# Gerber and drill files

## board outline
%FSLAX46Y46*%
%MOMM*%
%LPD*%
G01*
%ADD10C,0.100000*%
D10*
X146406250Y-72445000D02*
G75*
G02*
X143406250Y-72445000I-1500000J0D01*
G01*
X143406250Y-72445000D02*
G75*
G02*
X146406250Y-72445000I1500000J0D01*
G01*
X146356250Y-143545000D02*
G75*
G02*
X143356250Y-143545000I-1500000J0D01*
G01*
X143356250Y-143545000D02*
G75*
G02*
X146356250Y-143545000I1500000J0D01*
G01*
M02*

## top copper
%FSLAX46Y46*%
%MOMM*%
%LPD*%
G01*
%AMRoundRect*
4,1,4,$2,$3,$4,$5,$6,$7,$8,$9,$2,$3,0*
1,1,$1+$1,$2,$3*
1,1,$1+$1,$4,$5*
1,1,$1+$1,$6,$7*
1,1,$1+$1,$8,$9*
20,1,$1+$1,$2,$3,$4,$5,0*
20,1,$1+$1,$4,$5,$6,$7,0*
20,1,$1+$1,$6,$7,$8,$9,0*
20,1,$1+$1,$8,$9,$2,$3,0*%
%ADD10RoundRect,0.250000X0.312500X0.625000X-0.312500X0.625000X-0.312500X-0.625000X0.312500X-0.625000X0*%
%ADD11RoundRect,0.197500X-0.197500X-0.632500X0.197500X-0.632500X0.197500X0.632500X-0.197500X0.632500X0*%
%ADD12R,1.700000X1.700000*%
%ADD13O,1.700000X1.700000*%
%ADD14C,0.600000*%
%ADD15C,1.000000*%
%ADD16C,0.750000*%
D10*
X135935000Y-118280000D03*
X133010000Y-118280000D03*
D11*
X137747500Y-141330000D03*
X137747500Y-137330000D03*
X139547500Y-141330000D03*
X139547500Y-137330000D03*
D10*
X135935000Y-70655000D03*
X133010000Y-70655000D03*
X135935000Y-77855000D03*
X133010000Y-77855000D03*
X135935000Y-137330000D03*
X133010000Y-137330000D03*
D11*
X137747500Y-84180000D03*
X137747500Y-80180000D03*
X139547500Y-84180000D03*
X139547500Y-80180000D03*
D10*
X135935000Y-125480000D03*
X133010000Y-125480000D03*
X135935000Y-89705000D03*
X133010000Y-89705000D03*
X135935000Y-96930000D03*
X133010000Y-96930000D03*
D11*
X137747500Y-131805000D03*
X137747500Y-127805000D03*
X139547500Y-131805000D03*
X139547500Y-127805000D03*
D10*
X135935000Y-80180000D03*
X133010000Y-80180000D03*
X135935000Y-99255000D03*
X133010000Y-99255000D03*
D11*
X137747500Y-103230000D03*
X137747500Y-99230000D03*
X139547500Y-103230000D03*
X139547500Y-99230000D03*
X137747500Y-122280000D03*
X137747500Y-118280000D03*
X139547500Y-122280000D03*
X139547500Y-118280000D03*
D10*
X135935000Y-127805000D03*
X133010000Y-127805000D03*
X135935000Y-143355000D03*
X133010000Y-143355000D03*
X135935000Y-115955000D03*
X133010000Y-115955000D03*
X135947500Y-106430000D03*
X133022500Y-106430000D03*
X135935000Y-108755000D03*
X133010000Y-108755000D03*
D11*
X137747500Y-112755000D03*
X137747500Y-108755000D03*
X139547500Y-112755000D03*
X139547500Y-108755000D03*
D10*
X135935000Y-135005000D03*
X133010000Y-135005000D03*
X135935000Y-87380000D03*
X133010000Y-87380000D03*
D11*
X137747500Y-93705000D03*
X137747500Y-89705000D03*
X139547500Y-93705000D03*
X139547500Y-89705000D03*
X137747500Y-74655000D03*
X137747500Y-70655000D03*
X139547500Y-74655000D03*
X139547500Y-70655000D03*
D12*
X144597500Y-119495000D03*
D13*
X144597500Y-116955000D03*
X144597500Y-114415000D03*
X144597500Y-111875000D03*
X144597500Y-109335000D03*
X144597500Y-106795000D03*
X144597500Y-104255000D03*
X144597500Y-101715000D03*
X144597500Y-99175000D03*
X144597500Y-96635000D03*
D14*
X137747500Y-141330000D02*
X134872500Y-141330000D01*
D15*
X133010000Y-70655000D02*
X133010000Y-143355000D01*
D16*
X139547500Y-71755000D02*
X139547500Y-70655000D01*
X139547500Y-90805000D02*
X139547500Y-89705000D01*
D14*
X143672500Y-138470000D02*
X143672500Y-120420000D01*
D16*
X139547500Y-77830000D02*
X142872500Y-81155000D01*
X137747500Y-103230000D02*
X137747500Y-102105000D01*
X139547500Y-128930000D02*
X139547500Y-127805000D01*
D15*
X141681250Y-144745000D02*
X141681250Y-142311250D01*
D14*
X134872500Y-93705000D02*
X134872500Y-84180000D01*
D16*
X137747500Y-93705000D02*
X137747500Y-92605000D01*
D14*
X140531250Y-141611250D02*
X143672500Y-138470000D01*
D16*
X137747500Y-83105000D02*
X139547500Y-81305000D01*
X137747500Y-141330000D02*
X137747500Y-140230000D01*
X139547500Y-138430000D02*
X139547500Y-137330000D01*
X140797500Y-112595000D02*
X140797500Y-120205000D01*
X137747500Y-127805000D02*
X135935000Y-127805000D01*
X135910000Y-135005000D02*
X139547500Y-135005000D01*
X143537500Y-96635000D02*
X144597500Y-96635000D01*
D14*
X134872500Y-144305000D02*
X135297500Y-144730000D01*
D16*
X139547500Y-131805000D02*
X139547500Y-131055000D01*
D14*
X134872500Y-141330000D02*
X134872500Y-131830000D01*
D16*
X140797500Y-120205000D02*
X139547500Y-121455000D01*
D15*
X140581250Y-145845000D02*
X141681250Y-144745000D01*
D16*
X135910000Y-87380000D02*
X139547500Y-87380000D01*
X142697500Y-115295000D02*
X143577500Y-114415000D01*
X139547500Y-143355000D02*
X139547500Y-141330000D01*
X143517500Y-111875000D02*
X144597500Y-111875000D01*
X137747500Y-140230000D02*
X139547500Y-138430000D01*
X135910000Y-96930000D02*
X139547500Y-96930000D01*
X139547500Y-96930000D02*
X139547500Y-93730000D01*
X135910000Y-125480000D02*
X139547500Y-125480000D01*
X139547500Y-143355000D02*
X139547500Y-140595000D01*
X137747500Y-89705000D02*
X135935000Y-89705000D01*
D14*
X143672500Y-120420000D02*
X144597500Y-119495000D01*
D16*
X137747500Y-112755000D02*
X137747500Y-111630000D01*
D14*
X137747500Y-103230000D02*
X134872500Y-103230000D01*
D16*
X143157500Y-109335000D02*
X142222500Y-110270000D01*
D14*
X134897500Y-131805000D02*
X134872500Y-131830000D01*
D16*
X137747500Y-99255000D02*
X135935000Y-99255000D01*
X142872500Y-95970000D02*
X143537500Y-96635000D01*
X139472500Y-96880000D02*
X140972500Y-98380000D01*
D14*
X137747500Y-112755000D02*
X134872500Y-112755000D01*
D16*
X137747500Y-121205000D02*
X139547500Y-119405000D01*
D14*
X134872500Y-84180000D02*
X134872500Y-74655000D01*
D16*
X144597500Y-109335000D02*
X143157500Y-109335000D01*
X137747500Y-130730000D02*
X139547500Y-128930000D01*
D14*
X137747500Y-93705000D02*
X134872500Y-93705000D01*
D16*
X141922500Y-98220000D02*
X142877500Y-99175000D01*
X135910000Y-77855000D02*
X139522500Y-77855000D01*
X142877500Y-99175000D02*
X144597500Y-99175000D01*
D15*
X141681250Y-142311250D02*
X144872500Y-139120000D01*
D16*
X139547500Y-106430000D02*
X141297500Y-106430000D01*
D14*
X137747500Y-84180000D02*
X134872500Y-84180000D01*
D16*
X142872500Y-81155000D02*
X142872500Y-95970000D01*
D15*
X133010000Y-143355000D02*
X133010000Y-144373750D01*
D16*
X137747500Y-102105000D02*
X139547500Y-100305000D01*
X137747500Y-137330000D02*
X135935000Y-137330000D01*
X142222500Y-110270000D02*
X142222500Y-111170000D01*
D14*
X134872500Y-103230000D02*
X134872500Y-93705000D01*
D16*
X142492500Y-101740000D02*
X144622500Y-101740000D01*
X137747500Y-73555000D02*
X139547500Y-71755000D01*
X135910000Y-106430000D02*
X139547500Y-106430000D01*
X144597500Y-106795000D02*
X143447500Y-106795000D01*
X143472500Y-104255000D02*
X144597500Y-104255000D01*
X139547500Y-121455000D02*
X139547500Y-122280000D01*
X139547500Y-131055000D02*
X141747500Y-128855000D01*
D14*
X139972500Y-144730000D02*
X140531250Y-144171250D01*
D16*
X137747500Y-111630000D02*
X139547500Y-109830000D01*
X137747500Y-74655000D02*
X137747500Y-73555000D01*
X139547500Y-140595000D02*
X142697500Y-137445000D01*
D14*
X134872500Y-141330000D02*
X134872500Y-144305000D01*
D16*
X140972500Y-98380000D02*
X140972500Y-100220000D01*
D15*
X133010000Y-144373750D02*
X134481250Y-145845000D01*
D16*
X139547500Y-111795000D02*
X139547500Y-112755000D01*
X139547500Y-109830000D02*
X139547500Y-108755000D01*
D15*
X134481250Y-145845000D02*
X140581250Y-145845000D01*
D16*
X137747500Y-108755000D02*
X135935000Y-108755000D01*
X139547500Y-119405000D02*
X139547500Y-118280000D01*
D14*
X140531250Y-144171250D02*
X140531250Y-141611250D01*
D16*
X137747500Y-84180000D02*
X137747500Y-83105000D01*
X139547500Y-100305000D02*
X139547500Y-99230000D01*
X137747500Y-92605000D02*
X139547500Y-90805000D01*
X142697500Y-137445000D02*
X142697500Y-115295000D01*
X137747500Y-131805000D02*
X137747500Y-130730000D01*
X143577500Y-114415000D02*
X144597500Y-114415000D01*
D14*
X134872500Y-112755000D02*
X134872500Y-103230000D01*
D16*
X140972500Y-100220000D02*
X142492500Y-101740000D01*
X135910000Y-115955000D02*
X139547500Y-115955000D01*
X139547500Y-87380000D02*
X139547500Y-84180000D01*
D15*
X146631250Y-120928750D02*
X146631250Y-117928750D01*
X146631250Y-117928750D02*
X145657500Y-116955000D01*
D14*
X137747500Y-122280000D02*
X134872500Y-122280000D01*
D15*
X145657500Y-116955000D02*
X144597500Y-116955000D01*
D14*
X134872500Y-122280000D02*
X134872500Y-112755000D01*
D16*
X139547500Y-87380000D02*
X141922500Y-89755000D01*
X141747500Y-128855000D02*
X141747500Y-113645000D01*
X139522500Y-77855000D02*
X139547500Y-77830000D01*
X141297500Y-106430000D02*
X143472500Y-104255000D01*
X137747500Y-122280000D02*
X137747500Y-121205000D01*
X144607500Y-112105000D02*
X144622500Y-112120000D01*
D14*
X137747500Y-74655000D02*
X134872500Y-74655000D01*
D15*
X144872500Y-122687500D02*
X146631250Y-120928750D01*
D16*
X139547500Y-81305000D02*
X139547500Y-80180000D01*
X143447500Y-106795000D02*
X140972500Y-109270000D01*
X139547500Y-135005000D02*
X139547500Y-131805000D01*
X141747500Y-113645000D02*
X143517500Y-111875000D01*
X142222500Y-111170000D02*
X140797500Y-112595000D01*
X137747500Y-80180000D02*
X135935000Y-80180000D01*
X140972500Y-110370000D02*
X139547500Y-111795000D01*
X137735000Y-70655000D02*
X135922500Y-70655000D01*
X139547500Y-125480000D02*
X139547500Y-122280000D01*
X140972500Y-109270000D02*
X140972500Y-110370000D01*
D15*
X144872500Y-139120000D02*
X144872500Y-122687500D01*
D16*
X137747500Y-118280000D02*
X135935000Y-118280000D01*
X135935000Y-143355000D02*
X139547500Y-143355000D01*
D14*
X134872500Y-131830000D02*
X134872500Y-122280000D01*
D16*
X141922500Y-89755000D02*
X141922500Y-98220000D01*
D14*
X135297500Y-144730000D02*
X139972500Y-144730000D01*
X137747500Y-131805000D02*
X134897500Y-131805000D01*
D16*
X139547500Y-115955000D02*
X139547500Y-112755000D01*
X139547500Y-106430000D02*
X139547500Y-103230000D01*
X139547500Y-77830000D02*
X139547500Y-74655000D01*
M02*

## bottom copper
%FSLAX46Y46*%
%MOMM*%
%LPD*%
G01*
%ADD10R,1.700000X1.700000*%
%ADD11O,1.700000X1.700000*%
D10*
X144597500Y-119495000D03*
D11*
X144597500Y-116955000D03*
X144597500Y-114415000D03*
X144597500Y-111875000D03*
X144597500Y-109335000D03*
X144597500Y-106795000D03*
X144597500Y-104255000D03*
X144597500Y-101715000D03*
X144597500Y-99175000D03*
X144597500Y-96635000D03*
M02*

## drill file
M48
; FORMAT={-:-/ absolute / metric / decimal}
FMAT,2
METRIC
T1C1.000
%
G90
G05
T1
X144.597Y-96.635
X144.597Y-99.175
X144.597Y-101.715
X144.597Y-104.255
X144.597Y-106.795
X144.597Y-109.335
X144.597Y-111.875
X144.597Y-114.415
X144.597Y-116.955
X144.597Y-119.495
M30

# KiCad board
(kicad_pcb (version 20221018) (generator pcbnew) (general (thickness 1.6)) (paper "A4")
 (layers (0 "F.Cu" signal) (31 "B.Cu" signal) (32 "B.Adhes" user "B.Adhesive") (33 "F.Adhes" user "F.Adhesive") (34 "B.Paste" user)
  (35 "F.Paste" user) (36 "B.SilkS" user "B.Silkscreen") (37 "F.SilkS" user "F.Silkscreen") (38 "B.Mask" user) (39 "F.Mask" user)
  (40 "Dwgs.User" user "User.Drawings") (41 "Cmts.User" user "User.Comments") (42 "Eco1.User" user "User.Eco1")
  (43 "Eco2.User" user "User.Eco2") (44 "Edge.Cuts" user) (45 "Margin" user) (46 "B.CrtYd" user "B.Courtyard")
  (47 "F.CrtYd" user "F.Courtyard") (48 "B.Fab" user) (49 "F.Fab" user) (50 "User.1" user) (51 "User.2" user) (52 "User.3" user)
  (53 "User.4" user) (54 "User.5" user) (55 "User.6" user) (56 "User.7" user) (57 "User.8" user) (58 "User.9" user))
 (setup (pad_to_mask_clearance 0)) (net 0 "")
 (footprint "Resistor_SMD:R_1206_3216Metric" (layer "F.Cu") (at 134.4725 118.28 180)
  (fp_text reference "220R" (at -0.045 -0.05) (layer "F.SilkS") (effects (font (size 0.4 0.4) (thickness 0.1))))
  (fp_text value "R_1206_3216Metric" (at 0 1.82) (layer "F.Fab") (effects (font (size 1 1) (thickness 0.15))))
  (pad "1" smd roundrect (at -1.4625 0 180) (size 1.125 1.75) (layers "F.Cu" "F.Paste" "F.Mask") (roundrect_rratio 0.2222222222))
  (pad "2" smd roundrect (at 1.4625 0 180) (size 1.125 1.75) (layers "F.Cu" "F.Paste" "F.Mask") (roundrect_rratio 0.2222222222)))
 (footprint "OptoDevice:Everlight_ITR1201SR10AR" (layer "F.Cu") (at 138.6475 139.33)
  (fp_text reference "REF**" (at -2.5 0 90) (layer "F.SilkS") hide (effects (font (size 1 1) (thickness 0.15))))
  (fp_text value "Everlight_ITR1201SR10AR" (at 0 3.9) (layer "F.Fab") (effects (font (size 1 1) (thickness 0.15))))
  (pad "1" smd roundrect (at -0.9 2) (size 0.79 1.66) (layers "F.Cu" "F.Paste" "F.Mask") (roundrect_rratio 0.25))
  (pad "2" smd roundrect (at -0.9 -2) (size 0.79 1.66) (layers "F.Cu" "F.Paste" "F.Mask") (roundrect_rratio 0.25))
  (pad "3" smd roundrect (at 0.9 2) (size 0.79 1.66) (layers "F.Cu" "F.Paste" "F.Mask") (roundrect_rratio 0.25))
  (pad "4" smd roundrect (at 0.9 -2) (size 0.79 1.66) (layers "F.Cu" "F.Paste" "F.Mask") (roundrect_rratio 0.25)))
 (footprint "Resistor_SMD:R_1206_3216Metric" (layer "F.Cu") (at 134.4725 70.655 180)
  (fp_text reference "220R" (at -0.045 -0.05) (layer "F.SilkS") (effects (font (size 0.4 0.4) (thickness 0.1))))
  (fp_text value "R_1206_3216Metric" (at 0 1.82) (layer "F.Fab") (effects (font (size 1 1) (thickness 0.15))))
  (pad "1" smd roundrect (at -1.4625 0 180) (size 1.125 1.75) (layers "F.Cu" "F.Paste" "F.Mask") (roundrect_rratio 0.2222222222))
  (pad "2" smd roundrect (at 1.4625 0 180) (size 1.125 1.75) (layers "F.Cu" "F.Paste" "F.Mask") (roundrect_rratio 0.2222222222)))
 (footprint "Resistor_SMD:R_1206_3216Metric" (layer "F.Cu") (at 134.4725 77.855 180)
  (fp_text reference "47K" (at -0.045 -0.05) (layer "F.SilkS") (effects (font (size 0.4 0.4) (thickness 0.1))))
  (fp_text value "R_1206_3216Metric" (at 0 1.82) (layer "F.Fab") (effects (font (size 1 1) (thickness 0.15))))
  (pad "1" smd roundrect (at -1.4625 0 180) (size 1.125 1.75) (layers "F.Cu" "F.Paste" "F.Mask") (roundrect_rratio 0.2222222222))
  (pad "2" smd roundrect (at 1.4625 0 180) (size 1.125 1.75) (layers "F.Cu" "F.Paste" "F.Mask") (roundrect_rratio 0.2222222222)))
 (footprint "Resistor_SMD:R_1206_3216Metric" (layer "F.Cu") (at 134.4725 137.33 180)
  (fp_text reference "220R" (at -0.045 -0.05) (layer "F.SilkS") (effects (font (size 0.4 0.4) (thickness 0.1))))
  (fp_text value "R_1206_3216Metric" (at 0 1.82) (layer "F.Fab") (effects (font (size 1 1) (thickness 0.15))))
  (pad "1" smd roundrect (at -1.4625 0 180) (size 1.125 1.75) (layers "F.Cu" "F.Paste" "F.Mask") (roundrect_rratio 0.2222222222))
  (pad "2" smd roundrect (at 1.4625 0 180) (size 1.125 1.75) (layers "F.Cu" "F.Paste" "F.Mask") (roundrect_rratio 0.2222222222)))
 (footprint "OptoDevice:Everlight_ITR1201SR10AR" (layer "F.Cu") (at 138.6475 82.18)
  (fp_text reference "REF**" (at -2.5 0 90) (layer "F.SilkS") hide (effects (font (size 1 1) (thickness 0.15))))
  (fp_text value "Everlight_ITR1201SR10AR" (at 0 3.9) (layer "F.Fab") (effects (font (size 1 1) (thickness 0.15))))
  (pad "1" smd roundrect (at -0.9 2) (size 0.79 1.66) (layers "F.Cu" "F.Paste" "F.Mask") (roundrect_rratio 0.25))
  (pad "2" smd roundrect (at -0.9 -2) (size 0.79 1.66) (layers "F.Cu" "F.Paste" "F.Mask") (roundrect_rratio 0.25))
  (pad "3" smd roundrect (at 0.9 2) (size 0.79 1.66) (layers "F.Cu" "F.Paste" "F.Mask") (roundrect_rratio 0.25))
  (pad "4" smd roundrect (at 0.9 -2) (size 0.79 1.66) (layers "F.Cu" "F.Paste" "F.Mask") (roundrect_rratio 0.25)))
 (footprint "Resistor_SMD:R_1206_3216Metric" (layer "F.Cu") (at 134.4725 125.48 180)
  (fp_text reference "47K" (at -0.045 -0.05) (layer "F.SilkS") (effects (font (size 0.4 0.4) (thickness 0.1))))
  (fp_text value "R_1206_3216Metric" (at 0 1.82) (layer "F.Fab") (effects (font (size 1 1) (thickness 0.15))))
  (pad "1" smd roundrect (at -1.4625 0 180) (size 1.125 1.75) (layers "F.Cu" "F.Paste" "F.Mask") (roundrect_rratio 0.2222222222))
  (pad "2" smd roundrect (at 1.4625 0 180) (size 1.125 1.75) (layers "F.Cu" "F.Paste" "F.Mask") (roundrect_rratio 0.2222222222)))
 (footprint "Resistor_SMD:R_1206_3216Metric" (layer "F.Cu") (at 134.4725 89.705 180)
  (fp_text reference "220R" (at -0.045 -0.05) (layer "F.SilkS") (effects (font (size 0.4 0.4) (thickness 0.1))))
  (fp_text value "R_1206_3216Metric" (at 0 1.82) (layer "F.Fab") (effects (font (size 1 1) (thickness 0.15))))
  (pad "1" smd roundrect (at -1.4625 0 180) (size 1.125 1.75) (layers "F.Cu" "F.Paste" "F.Mask") (roundrect_rratio 0.2222222222))
  (pad "2" smd roundrect (at 1.4625 0 180) (size 1.125 1.75) (layers "F.Cu" "F.Paste" "F.Mask") (roundrect_rratio 0.2222222222)))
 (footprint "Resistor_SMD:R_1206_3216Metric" (layer "F.Cu") (at 134.4725 96.93 180)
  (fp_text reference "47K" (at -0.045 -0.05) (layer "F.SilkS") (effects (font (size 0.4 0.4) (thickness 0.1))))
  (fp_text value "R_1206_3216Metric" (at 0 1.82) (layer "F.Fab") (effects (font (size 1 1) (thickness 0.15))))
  (pad "1" smd roundrect (at -1.4625 0 180) (size 1.125 1.75) (layers "F.Cu" "F.Paste" "F.Mask") (roundrect_rratio 0.2222222222))
  (pad "2" smd roundrect (at 1.4625 0 180) (size 1.125 1.75) (layers "F.Cu" "F.Paste" "F.Mask") (roundrect_rratio 0.2222222222)))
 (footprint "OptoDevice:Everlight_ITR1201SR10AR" (layer "F.Cu") (at 138.6475 129.805)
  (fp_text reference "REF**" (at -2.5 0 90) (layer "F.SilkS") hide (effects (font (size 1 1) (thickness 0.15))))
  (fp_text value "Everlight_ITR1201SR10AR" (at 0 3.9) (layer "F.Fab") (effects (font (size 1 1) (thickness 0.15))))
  (pad "1" smd roundrect (at -0.9 2) (size 0.79 1.66) (layers "F.Cu" "F.Paste" "F.Mask") (roundrect_rratio 0.25))
  (pad "2" smd roundrect (at -0.9 -2) (size 0.79 1.66) (layers "F.Cu" "F.Paste" "F.Mask") (roundrect_rratio 0.25))
  (pad "3" smd roundrect (at 0.9 2) (size 0.79 1.66) (layers "F.Cu" "F.Paste" "F.Mask") (roundrect_rratio 0.25))
  (pad "4" smd roundrect (at 0.9 -2) (size 0.79 1.66) (layers "F.Cu" "F.Paste" "F.Mask") (roundrect_rratio 0.25)))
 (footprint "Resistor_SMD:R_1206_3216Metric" (layer "F.Cu") (at 134.4725 80.18 180)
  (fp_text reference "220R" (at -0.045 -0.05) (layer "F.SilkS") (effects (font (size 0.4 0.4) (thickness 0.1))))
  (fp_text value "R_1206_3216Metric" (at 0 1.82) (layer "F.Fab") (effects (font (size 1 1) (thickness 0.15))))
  (pad "1" smd roundrect (at -1.4625 0 180) (size 1.125 1.75) (layers "F.Cu" "F.Paste" "F.Mask") (roundrect_rratio 0.2222222222))
  (pad "2" smd roundrect (at 1.4625 0 180) (size 1.125 1.75) (layers "F.Cu" "F.Paste" "F.Mask") (roundrect_rratio 0.2222222222)))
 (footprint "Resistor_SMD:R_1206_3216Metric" (layer "F.Cu") (at 134.4725 99.255 180)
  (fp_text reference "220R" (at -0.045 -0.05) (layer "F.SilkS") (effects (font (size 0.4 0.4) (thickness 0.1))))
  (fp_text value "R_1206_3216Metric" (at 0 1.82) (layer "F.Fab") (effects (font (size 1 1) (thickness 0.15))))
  (pad "1" smd roundrect (at -1.4625 0 180) (size 1.125 1.75) (layers "F.Cu" "F.Paste" "F.Mask") (roundrect_rratio 0.2222222222))
  (pad "2" smd roundrect (at 1.4625 0 180) (size 1.125 1.75) (layers "F.Cu" "F.Paste" "F.Mask") (roundrect_rratio 0.2222222222)))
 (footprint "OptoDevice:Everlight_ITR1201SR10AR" (layer "F.Cu") (at 138.6475 101.23)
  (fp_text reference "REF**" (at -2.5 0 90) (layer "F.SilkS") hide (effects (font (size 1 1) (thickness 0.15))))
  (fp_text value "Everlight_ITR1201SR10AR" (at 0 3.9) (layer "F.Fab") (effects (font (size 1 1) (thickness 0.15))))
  (pad "1" smd roundrect (at -0.9 2) (size 0.79 1.66) (layers "F.Cu" "F.Paste" "F.Mask") (roundrect_rratio 0.25))
  (pad "2" smd roundrect (at -0.9 -2) (size 0.79 1.66) (layers "F.Cu" "F.Paste" "F.Mask") (roundrect_rratio 0.25))
  (pad "3" smd roundrect (at 0.9 2) (size 0.79 1.66) (layers "F.Cu" "F.Paste" "F.Mask") (roundrect_rratio 0.25))
  (pad "4" smd roundrect (at 0.9 -2) (size 0.79 1.66) (layers "F.Cu" "F.Paste" "F.Mask") (roundrect_rratio 0.25)))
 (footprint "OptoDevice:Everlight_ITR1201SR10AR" (layer "F.Cu") (at 138.6475 120.28)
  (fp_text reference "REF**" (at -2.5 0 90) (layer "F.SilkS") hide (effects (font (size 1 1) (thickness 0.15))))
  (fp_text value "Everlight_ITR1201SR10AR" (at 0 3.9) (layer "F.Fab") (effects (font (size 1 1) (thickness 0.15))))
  (pad "1" smd roundrect (at -0.9 2) (size 0.79 1.66) (layers "F.Cu" "F.Paste" "F.Mask") (roundrect_rratio 0.25))
  (pad "2" smd roundrect (at -0.9 -2) (size 0.79 1.66) (layers "F.Cu" "F.Paste" "F.Mask") (roundrect_rratio 0.25))
  (pad "3" smd roundrect (at 0.9 2) (size 0.79 1.66) (layers "F.Cu" "F.Paste" "F.Mask") (roundrect_rratio 0.25))
  (pad "4" smd roundrect (at 0.9 -2) (size 0.79 1.66) (layers "F.Cu" "F.Paste" "F.Mask") (roundrect_rratio 0.25)))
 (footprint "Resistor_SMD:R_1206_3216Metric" (layer "F.Cu") (at 134.4725 127.805 180)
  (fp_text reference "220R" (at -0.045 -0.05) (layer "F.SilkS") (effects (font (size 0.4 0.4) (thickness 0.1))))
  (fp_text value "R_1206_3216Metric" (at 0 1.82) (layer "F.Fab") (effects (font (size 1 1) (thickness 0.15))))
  (pad "1" smd roundrect (at -1.4625 0 180) (size 1.125 1.75) (layers "F.Cu" "F.Paste" "F.Mask") (roundrect_rratio 0.2222222222))
  (pad "2" smd roundrect (at 1.4625 0 180) (size 1.125 1.75) (layers "F.Cu" "F.Paste" "F.Mask") (roundrect_rratio 0.2222222222)))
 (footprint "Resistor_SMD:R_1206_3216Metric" (layer "F.Cu") (at 134.4725 143.355 180)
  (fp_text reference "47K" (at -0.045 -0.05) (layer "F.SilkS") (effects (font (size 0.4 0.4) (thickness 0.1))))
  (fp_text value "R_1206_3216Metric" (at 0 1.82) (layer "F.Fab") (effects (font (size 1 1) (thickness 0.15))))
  (pad "1" smd roundrect (at -1.4625 0 180) (size 1.125 1.75) (layers "F.Cu" "F.Paste" "F.Mask") (roundrect_rratio 0.2222222222))
  (pad "2" smd roundrect (at 1.4625 0 180) (size 1.125 1.75) (layers "F.Cu" "F.Paste" "F.Mask") (roundrect_rratio 0.2222222222)))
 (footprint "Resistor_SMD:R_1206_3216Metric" (layer "F.Cu") (at 134.4725 115.955 180)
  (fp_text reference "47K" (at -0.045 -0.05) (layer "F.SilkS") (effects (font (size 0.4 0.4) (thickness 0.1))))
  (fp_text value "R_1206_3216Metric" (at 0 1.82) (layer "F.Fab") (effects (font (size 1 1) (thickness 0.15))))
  (pad "1" smd roundrect (at -1.4625 0 180) (size 1.125 1.75) (layers "F.Cu" "F.Paste" "F.Mask") (roundrect_rratio 0.2222222222))
  (pad "2" smd roundrect (at 1.4625 0 180) (size 1.125 1.75) (layers "F.Cu" "F.Paste" "F.Mask") (roundrect_rratio 0.2222222222)))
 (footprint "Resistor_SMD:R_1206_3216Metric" (layer "F.Cu") (at 134.485 106.43 180)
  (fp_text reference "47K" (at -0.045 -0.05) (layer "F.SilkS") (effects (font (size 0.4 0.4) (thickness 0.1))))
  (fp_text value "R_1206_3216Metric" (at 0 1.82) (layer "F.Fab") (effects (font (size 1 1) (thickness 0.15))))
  (pad "1" smd roundrect (at -1.4625 0 180) (size 1.125 1.75) (layers "F.Cu" "F.Paste" "F.Mask") (roundrect_rratio 0.2222222222))
  (pad "2" smd roundrect (at 1.4625 0 180) (size 1.125 1.75) (layers "F.Cu" "F.Paste" "F.Mask") (roundrect_rratio 0.2222222222)))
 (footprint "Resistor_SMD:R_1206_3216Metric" (layer "F.Cu") (at 134.4725 108.755 180)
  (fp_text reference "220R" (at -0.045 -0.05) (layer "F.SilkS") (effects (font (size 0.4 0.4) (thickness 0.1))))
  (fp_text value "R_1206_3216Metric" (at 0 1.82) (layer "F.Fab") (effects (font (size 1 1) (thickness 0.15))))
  (pad "1" smd roundrect (at -1.4625 0 180) (size 1.125 1.75) (layers "F.Cu" "F.Paste" "F.Mask") (roundrect_rratio 0.2222222222))
  (pad "2" smd roundrect (at 1.4625 0 180) (size 1.125 1.75) (layers "F.Cu" "F.Paste" "F.Mask") (roundrect_rratio 0.2222222222)))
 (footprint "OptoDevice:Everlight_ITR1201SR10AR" (layer "F.Cu") (at 138.6475 110.755)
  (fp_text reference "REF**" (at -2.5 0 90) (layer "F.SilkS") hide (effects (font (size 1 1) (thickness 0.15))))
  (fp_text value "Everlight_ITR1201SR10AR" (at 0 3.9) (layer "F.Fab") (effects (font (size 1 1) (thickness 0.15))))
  (pad "1" smd roundrect (at -0.9 2) (size 0.79 1.66) (layers "F.Cu" "F.Paste" "F.Mask") (roundrect_rratio 0.25))
  (pad "2" smd roundrect (at -0.9 -2) (size 0.79 1.66) (layers "F.Cu" "F.Paste" "F.Mask") (roundrect_rratio 0.25))
  (pad "3" smd roundrect (at 0.9 2) (size 0.79 1.66) (layers "F.Cu" "F.Paste" "F.Mask") (roundrect_rratio 0.25))
  (pad "4" smd roundrect (at 0.9 -2) (size 0.79 1.66) (layers "F.Cu" "F.Paste" "F.Mask") (roundrect_rratio 0.25)))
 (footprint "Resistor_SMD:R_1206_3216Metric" (layer "F.Cu") (at 134.4725 135.005 180)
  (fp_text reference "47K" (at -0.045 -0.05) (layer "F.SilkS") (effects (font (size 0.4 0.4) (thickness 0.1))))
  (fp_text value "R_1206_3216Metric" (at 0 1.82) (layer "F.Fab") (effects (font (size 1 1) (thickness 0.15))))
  (pad "1" smd roundrect (at -1.4625 0 180) (size 1.125 1.75) (layers "F.Cu" "F.Paste" "F.Mask") (roundrect_rratio 0.2222222222))
  (pad "2" smd roundrect (at 1.4625 0 180) (size 1.125 1.75) (layers "F.Cu" "F.Paste" "F.Mask") (roundrect_rratio 0.2222222222)))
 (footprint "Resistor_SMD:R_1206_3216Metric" (layer "F.Cu") (at 134.4725 87.38 180)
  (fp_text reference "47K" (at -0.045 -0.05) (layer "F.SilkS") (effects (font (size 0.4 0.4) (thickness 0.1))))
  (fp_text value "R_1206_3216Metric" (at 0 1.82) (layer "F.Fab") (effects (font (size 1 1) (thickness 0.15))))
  (pad "1" smd roundrect (at -1.4625 0 180) (size 1.125 1.75) (layers "F.Cu" "F.Paste" "F.Mask") (roundrect_rratio 0.2222222222))
  (pad "2" smd roundrect (at 1.4625 0 180) (size 1.125 1.75) (layers "F.Cu" "F.Paste" "F.Mask") (roundrect_rratio 0.2222222222)))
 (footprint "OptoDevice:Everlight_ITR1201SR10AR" (layer "F.Cu") (at 138.6475 91.705)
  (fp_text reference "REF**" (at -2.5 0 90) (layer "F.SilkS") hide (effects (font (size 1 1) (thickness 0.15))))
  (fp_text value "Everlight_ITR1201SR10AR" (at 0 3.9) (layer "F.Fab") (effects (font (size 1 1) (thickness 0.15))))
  (pad "1" smd roundrect (at -0.9 2) (size 0.79 1.66) (layers "F.Cu" "F.Paste" "F.Mask") (roundrect_rratio 0.25))
  (pad "2" smd roundrect (at -0.9 -2) (size 0.79 1.66) (layers "F.Cu" "F.Paste" "F.Mask") (roundrect_rratio 0.25))
  (pad "3" smd roundrect (at 0.9 2) (size 0.79 1.66) (layers "F.Cu" "F.Paste" "F.Mask") (roundrect_rratio 0.25))
  (pad "4" smd roundrect (at 0.9 -2) (size 0.79 1.66) (layers "F.Cu" "F.Paste" "F.Mask") (roundrect_rratio 0.25)))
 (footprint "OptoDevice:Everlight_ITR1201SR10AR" (layer "F.Cu") (at 138.6475 72.655)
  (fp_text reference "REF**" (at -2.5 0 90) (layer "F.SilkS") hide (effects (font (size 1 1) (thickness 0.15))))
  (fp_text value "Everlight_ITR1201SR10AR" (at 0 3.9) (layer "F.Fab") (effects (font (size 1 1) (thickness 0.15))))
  (pad "1" smd roundrect (at -0.9 2) (size 0.79 1.66) (layers "F.Cu" "F.Paste" "F.Mask") (roundrect_rratio 0.25))
  (pad "2" smd roundrect (at -0.9 -2) (size 0.79 1.66) (layers "F.Cu" "F.Paste" "F.Mask") (roundrect_rratio 0.25))
  (pad "3" smd roundrect (at 0.9 2) (size 0.79 1.66) (layers "F.Cu" "F.Paste" "F.Mask") (roundrect_rratio 0.25))
  (pad "4" smd roundrect (at 0.9 -2) (size 0.79 1.66) (layers "F.Cu" "F.Paste" "F.Mask") (roundrect_rratio 0.25)))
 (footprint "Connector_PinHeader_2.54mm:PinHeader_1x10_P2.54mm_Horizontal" (layer "B.Cu") (at 144.5975 119.495)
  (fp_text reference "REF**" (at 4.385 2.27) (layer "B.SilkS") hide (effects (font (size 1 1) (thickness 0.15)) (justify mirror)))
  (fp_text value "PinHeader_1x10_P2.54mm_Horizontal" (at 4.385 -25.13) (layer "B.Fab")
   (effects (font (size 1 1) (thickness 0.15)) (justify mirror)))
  (pad "1" thru_hole rect (at 0 0) (size 1.7 1.7) (drill 1) (layers "*.Cu" "*.Mask"))
  (pad "2" thru_hole oval (at 0 -2.54) (size 1.7 1.7) (drill 1) (layers "*.Cu" "*.Mask"))
  (pad "3" thru_hole oval (at 0 -5.08) (size 1.7 1.7) (drill 1) (layers "*.Cu" "*.Mask"))
  (pad "4" thru_hole oval (at 0 -7.62) (size 1.7 1.7) (drill 1) (layers "*.Cu" "*.Mask"))
  (pad "5" thru_hole oval (at 0 -10.16) (size 1.7 1.7) (drill 1) (layers "*.Cu" "*.Mask"))
  (pad "6" thru_hole oval (at 0 -12.7) (size 1.7 1.7) (drill 1) (layers "*.Cu" "*.Mask"))
  (pad "7" thru_hole oval (at 0 -15.24) (size 1.7 1.7) (drill 1) (layers "*.Cu" "*.Mask"))
  (pad "8" thru_hole oval (at 0 -17.78) (size 1.7 1.7) (drill 1) (layers "*.Cu" "*.Mask"))
  (pad "9" thru_hole oval (at 0 -20.32) (size 1.7 1.7) (drill 1) (layers "*.Cu" "*.Mask"))
  (pad "10" thru_hole oval (at 0 -22.86) (size 1.7 1.7) (drill 1) (layers "*.Cu" "*.Mask")))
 (gr_circle (center 144.90625 72.445) (end 143.40625 72.445) (stroke (width 0.1) (type solid)) (fill none) (layer "Edge.Cuts"))
 (gr_circle (center 144.85625 143.545) (end 146.35625 143.545) (stroke (width 0.1) (type solid)) (fill none) (layer "Edge.Cuts"))
 (segment (start 137.7475 141.33) (end 134.8725 141.33) (width 0.6) (layer "F.Cu") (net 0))
 (segment (start 133.01 70.655) (end 133.01 143.355) (width 1) (layer "F.Cu") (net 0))
 (segment (start 139.5475 71.755) (end 139.5475 70.655) (width 0.75) (layer "F.Cu") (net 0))
 (segment (start 139.5475 90.805) (end 139.5475 89.705) (width 0.75) (layer "F.Cu") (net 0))
 (segment (start 143.6725 138.47) (end 143.6725 120.42) (width 0.6) (layer "F.Cu") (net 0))
 (segment (start 139.5475 77.83) (end 142.8725 81.155) (width 0.75) (layer "F.Cu") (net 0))
 (segment (start 137.7475 103.23) (end 137.7475 102.105) (width 0.75) (layer "F.Cu") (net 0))
 (segment (start 139.5475 128.93) (end 139.5475 127.805) (width 0.75) (layer "F.Cu") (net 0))
 (segment (start 141.68125 144.745) (end 141.68125 142.31125) (width 1) (layer "F.Cu") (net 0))
 (segment (start 134.8725 93.705) (end 134.8725 84.18) (width 0.6) (layer "F.Cu") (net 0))
 (segment (start 137.7475 93.705) (end 137.7475 92.605) (width 0.75) (layer "F.Cu") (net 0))
 (segment (start 140.53125 141.61125) (end 143.6725 138.47) (width 0.6) (layer "F.Cu") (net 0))
 (segment (start 137.7475 83.105) (end 139.5475 81.305) (width 0.75) (layer "F.Cu") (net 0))
 (segment (start 137.7475 141.33) (end 137.7475 140.23) (width 0.75) (layer "F.Cu") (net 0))
 (segment (start 139.5475 138.43) (end 139.5475 137.33) (width 0.75) (layer "F.Cu") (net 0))
 (segment (start 140.7975 112.595) (end 140.7975 120.205) (width 0.75) (layer "F.Cu") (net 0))
 (segment (start 137.7475 127.805) (end 135.935 127.805) (width 0.75) (layer "F.Cu") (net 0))
 (segment (start 135.91 135.005) (end 139.5475 135.005) (width 0.75) (layer "F.Cu") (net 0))
 (segment (start 143.5375 96.635) (end 144.5975 96.635) (width 0.75) (layer "F.Cu") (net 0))
 (segment (start 134.8725 144.305) (end 135.2975 144.73) (width 0.6) (layer "F.Cu") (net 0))
 (segment (start 139.5475 131.805) (end 139.5475 131.055) (width 0.75) (layer "F.Cu") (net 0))
 (segment (start 134.8725 141.33) (end 134.8725 131.83) (width 0.6) (layer "F.Cu") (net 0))
 (segment (start 140.7975 120.205) (end 139.5475 121.455) (width 0.75) (layer "F.Cu") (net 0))
 (segment (start 140.58125 145.845) (end 141.68125 144.745) (width 1) (layer "F.Cu") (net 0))
 (segment (start 135.91 87.38) (end 139.5475 87.38) (width 0.75) (layer "F.Cu") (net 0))
 (segment (start 142.6975 115.295) (end 143.5775 114.415) (width 0.75) (layer "F.Cu") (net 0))
 (segment (start 139.5475 143.355) (end 139.5475 141.33) (width 0.75) (layer "F.Cu") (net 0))
 (segment (start 143.5175 111.875) (end 144.5975 111.875) (width 0.75) (layer "F.Cu") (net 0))
 (segment (start 137.7475 140.23) (end 139.5475 138.43) (width 0.75) (layer "F.Cu") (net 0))
 (segment (start 135.91 96.93) (end 139.5475 96.93) (width 0.75) (layer "F.Cu") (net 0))
 (segment (start 139.5475 96.93) (end 139.5475 93.73) (width 0.75) (layer "F.Cu") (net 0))
 (segment (start 135.91 125.48) (end 139.5475 125.48) (width 0.75) (layer "F.Cu") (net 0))
 (segment (start 139.5475 143.355) (end 139.5475 140.595) (width 0.75) (layer "F.Cu") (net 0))
 (segment (start 137.7475 89.705) (end 135.935 89.705) (width 0.75) (layer "F.Cu") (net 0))
 (segment (start 143.6725 120.42) (end 144.5975 119.495) (width 0.6) (layer "F.Cu") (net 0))
 (segment (start 137.7475 112.755) (end 137.7475 111.63) (width 0.75) (layer "F.Cu") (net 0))
 (segment (start 137.7475 103.23) (end 134.8725 103.23) (width 0.6) (layer "F.Cu") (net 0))
 (segment (start 143.1575 109.335) (end 142.2225 110.27) (width 0.75) (layer "F.Cu") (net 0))
 (segment (start 134.8975 131.805) (end 134.8725 131.83) (width 0.6) (layer "F.Cu") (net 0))
 (segment (start 137.7475 99.255) (end 135.935 99.255) (width 0.75) (layer "F.Cu") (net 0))
 (segment (start 142.8725 95.97) (end 143.5375 96.635) (width 0.75) (layer "F.Cu") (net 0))
 (segment (start 139.4725 96.88) (end 140.9725 98.38) (width 0.75) (layer "F.Cu") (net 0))
 (segment (start 137.7475 112.755) (end 134.8725 112.755) (width 0.6) (layer "F.Cu") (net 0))
 (segment (start 137.7475 121.205) (end 139.5475 119.405) (width 0.75) (layer "F.Cu") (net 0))
 (segment (start 134.8725 84.18) (end 134.8725 74.655) (width 0.6) (layer "F.Cu") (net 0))
 (segment (start 144.5975 109.335) (end 143.1575 109.335) (width 0.75) (layer "F.Cu") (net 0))
 (segment (start 137.7475 130.73) (end 139.5475 128.93) (width 0.75) (layer "F.Cu") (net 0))
 (segment (start 137.7475 93.705) (end 134.8725 93.705) (width 0.6) (layer "F.Cu") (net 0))
 (segment (start 141.9225 98.22) (end 142.8775 99.175) (width 0.75) (layer "F.Cu") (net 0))
 (segment (start 135.91 77.855) (end 139.5225 77.855) (width 0.75) (layer "F.Cu") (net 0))
 (segment (start 142.8775 99.175) (end 144.5975 99.175) (width 0.75) (layer "F.Cu") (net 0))
 (segment (start 141.68125 142.31125) (end 144.8725 139.12) (width 1) (layer "F.Cu") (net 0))
 (segment (start 139.5475 106.43) (end 141.2975 106.43) (width 0.75) (layer "F.Cu") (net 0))
 (segment (start 137.7475 84.18) (end 134.8725 84.18) (width 0.6) (layer "F.Cu") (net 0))
 (segment (start 142.8725 81.155) (end 142.8725 95.97) (width 0.75) (layer "F.Cu") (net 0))
 (segment (start 133.01 143.355) (end 133.01 144.37375) (width 1) (layer "F.Cu") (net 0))
 (segment (start 137.7475 102.105) (end 139.5475 100.305) (width 0.75) (layer "F.Cu") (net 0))
 (segment (start 137.7475 137.33) (end 135.935 137.33) (width 0.75) (layer "F.Cu") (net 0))
 (segment (start 142.2225 110.27) (end 142.2225 111.17) (width 0.75) (layer "F.Cu") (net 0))
 (segment (start 134.8725 103.23) (end 134.8725 93.705) (width 0.6) (layer "F.Cu") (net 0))
 (segment (start 142.4925 101.74) (end 144.6225 101.74) (width 0.75) (layer "F.Cu") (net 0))
 (segment (start 137.7475 73.555) (end 139.5475 71.755) (width 0.75) (layer "F.Cu") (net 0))
 (segment (start 135.91 106.43) (end 139.5475 106.43) (width 0.75) (layer "F.Cu") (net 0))
 (segment (start 144.5975 106.795) (end 143.4475 106.795) (width 0.75) (layer "F.Cu") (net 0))
 (segment (start 143.4725 104.255) (end 144.5975 104.255) (width 0.75) (layer "F.Cu") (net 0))
 (segment (start 139.5475 121.455) (end 139.5475 122.28) (width 0.75) (layer "F.Cu") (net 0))
 (segment (start 139.5475 131.055) (end 141.7475 128.855) (width 0.75) (layer "F.Cu") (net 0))
 (segment (start 139.9725 144.73) (end 140.53125 144.17125) (width 0.6) (layer "F.Cu") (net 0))
 (segment (start 137.7475 111.63) (end 139.5475 109.83) (width 0.75) (layer "F.Cu") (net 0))
 (segment (start 137.7475 74.655) (end 137.7475 73.555) (width 0.75) (layer "F.Cu") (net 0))
 (segment (start 139.5475 140.595) (end 142.6975 137.445) (width 0.75) (layer "F.Cu") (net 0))
 (segment (start 134.8725 141.33) (end 134.8725 144.305) (width 0.6) (layer "F.Cu") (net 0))
 (segment (start 140.9725 98.38) (end 140.9725 100.22) (width 0.75) (layer "F.Cu") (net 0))
 (segment (start 133.01 144.37375) (end 134.48125 145.845) (width 1) (layer "F.Cu") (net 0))
 (segment (start 139.5475 111.795) (end 139.5475 112.755) (width 0.75) (layer "F.Cu") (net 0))
 (segment (start 139.5475 109.83) (end 139.5475 108.755) (width 0.75) (layer "F.Cu") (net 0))
 (segment (start 134.48125 145.845) (end 140.58125 145.845) (width 1) (layer "F.Cu") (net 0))
 (segment (start 137.7475 108.755) (end 135.935 108.755) (width 0.75) (layer "F.Cu") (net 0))
 (segment (start 139.5475 119.405) (end 139.5475 118.28) (width 0.75) (layer "F.Cu") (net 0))
 (segment (start 140.53125 144.17125) (end 140.53125 141.61125) (width 0.6) (layer "F.Cu") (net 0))
 (segment (start 137.7475 84.18) (end 137.7475 83.105) (width 0.75) (layer "F.Cu") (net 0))
 (segment (start 139.5475 100.305) (end 139.5475 99.23) (width 0.75) (layer "F.Cu") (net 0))
 (segment (start 137.7475 92.605) (end 139.5475 90.805) (width 0.75) (layer "F.Cu") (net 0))
 (segment (start 142.6975 137.445) (end 142.6975 115.295) (width 0.75) (layer "F.Cu") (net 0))
 (segment (start 137.7475 131.805) (end 137.7475 130.73) (width 0.75) (layer "F.Cu") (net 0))
 (segment (start 143.5775 114.415) (end 144.5975 114.415) (width 0.75) (layer "F.Cu") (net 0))
 (segment (start 134.8725 112.755) (end 134.8725 103.23) (width 0.6) (layer "F.Cu") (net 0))
 (segment (start 140.9725 100.22) (end 142.4925 101.74) (width 0.75) (layer "F.Cu") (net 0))
 (segment (start 135.91 115.955) (end 139.5475 115.955) (width 0.75) (layer "F.Cu") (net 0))
 (segment (start 139.5475 87.38) (end 139.5475 84.18) (width 0.75) (layer "F.Cu") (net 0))
 (segment (start 146.63125 120.92875) (end 146.63125 117.92875) (width 1) (layer "F.Cu") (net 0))
 (segment (start 146.63125 117.92875) (end 145.6575 116.955) (width 1) (layer "F.Cu") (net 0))
 (segment (start 137.7475 122.28) (end 134.8725 122.28) (width 0.6) (layer "F.Cu") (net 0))
 (segment (start 145.6575 116.955) (end 144.5975 116.955) (width 1) (layer "F.Cu") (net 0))
 (segment (start 134.8725 122.28) (end 134.8725 112.755) (width 0.6) (layer "F.Cu") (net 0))
 (segment (start 139.5475 87.38) (end 141.9225 89.755) (width 0.75) (layer "F.Cu") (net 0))
 (segment (start 141.7475 128.855) (end 141.7475 113.645) (width 0.75) (layer "F.Cu") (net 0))
 (segment (start 139.5225 77.855) (end 139.5475 77.83) (width 0.75) (layer "F.Cu") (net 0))
 (segment (start 141.2975 106.43) (end 143.4725 104.255) (width 0.75) (layer "F.Cu") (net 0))
 (segment (start 137.7475 122.28) (end 137.7475 121.205) (width 0.75) (layer "F.Cu") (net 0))
 (segment (start 144.6075 112.105) (end 144.6225 112.12) (width 0.75) (layer "F.Cu") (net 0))
 (segment (start 137.7475 74.655) (end 134.8725 74.655) (width 0.6) (layer "F.Cu") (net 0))
 (segment (start 144.8725 122.6875) (end 146.63125 120.92875) (width 1) (layer "F.Cu") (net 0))
 (segment (start 139.5475 81.305) (end 139.5475 80.18) (width 0.75) (layer "F.Cu") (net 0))
 (segment (start 143.4475 106.795) (end 140.9725 109.27) (width 0.75) (layer "F.Cu") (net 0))
 (segment (start 139.5475 135.005) (end 139.5475 131.805) (width 0.75) (layer "F.Cu") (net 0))
 (segment (start 141.7475 113.645) (end 143.5175 111.875) (width 0.75) (layer "F.Cu") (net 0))
 (segment (start 142.2225 111.17) (end 140.7975 112.595) (width 0.75) (layer "F.Cu") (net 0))
 (segment (start 137.7475 80.18) (end 135.935 80.18) (width 0.75) (layer "F.Cu") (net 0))
 (segment (start 140.9725 110.37) (end 139.5475 111.795) (width 0.75) (layer "F.Cu") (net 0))
 (segment (start 137.735 70.655) (end 135.9225 70.655) (width 0.75) (layer "F.Cu") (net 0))
 (segment (start 139.5475 125.48) (end 139.5475 122.28) (width 0.75) (layer "F.Cu") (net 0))
 (segment (start 140.9725 109.27) (end 140.9725 110.37) (width 0.75) (layer "F.Cu") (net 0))
 (segment (start 144.8725 139.12) (end 144.8725 122.6875) (width 1) (layer "F.Cu") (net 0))
 (segment (start 137.7475 118.28) (end 135.935 118.28) (width 0.75) (layer "F.Cu") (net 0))
 (segment (start 135.935 143.355) (end 139.5475 143.355) (width 0.75) (layer "F.Cu") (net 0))
 (segment (start 134.8725 131.83) (end 134.8725 122.28) (width 0.6) (layer "F.Cu") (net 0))
 (segment (start 141.9225 89.755) (end 141.9225 98.22) (width 0.75) (layer "F.Cu") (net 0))
 (segment (start 135.2975 144.73) (end 139.9725 144.73) (width 0.6) (layer "F.Cu") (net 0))
 (segment (start 137.7475 131.805) (end 134.8975 131.805) (width 0.6) (layer "F.Cu") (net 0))
 (segment (start 139.5475 115.955) (end 139.5475 112.755) (width 0.75) (layer "F.Cu") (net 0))
 (segment (start 139.5475 106.43) (end 139.5475 103.23) (width 0.75) (layer "F.Cu") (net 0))
 (segment (start 139.5475 77.83) (end 139.5475 74.655) (width 0.75) (layer "F.Cu") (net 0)))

